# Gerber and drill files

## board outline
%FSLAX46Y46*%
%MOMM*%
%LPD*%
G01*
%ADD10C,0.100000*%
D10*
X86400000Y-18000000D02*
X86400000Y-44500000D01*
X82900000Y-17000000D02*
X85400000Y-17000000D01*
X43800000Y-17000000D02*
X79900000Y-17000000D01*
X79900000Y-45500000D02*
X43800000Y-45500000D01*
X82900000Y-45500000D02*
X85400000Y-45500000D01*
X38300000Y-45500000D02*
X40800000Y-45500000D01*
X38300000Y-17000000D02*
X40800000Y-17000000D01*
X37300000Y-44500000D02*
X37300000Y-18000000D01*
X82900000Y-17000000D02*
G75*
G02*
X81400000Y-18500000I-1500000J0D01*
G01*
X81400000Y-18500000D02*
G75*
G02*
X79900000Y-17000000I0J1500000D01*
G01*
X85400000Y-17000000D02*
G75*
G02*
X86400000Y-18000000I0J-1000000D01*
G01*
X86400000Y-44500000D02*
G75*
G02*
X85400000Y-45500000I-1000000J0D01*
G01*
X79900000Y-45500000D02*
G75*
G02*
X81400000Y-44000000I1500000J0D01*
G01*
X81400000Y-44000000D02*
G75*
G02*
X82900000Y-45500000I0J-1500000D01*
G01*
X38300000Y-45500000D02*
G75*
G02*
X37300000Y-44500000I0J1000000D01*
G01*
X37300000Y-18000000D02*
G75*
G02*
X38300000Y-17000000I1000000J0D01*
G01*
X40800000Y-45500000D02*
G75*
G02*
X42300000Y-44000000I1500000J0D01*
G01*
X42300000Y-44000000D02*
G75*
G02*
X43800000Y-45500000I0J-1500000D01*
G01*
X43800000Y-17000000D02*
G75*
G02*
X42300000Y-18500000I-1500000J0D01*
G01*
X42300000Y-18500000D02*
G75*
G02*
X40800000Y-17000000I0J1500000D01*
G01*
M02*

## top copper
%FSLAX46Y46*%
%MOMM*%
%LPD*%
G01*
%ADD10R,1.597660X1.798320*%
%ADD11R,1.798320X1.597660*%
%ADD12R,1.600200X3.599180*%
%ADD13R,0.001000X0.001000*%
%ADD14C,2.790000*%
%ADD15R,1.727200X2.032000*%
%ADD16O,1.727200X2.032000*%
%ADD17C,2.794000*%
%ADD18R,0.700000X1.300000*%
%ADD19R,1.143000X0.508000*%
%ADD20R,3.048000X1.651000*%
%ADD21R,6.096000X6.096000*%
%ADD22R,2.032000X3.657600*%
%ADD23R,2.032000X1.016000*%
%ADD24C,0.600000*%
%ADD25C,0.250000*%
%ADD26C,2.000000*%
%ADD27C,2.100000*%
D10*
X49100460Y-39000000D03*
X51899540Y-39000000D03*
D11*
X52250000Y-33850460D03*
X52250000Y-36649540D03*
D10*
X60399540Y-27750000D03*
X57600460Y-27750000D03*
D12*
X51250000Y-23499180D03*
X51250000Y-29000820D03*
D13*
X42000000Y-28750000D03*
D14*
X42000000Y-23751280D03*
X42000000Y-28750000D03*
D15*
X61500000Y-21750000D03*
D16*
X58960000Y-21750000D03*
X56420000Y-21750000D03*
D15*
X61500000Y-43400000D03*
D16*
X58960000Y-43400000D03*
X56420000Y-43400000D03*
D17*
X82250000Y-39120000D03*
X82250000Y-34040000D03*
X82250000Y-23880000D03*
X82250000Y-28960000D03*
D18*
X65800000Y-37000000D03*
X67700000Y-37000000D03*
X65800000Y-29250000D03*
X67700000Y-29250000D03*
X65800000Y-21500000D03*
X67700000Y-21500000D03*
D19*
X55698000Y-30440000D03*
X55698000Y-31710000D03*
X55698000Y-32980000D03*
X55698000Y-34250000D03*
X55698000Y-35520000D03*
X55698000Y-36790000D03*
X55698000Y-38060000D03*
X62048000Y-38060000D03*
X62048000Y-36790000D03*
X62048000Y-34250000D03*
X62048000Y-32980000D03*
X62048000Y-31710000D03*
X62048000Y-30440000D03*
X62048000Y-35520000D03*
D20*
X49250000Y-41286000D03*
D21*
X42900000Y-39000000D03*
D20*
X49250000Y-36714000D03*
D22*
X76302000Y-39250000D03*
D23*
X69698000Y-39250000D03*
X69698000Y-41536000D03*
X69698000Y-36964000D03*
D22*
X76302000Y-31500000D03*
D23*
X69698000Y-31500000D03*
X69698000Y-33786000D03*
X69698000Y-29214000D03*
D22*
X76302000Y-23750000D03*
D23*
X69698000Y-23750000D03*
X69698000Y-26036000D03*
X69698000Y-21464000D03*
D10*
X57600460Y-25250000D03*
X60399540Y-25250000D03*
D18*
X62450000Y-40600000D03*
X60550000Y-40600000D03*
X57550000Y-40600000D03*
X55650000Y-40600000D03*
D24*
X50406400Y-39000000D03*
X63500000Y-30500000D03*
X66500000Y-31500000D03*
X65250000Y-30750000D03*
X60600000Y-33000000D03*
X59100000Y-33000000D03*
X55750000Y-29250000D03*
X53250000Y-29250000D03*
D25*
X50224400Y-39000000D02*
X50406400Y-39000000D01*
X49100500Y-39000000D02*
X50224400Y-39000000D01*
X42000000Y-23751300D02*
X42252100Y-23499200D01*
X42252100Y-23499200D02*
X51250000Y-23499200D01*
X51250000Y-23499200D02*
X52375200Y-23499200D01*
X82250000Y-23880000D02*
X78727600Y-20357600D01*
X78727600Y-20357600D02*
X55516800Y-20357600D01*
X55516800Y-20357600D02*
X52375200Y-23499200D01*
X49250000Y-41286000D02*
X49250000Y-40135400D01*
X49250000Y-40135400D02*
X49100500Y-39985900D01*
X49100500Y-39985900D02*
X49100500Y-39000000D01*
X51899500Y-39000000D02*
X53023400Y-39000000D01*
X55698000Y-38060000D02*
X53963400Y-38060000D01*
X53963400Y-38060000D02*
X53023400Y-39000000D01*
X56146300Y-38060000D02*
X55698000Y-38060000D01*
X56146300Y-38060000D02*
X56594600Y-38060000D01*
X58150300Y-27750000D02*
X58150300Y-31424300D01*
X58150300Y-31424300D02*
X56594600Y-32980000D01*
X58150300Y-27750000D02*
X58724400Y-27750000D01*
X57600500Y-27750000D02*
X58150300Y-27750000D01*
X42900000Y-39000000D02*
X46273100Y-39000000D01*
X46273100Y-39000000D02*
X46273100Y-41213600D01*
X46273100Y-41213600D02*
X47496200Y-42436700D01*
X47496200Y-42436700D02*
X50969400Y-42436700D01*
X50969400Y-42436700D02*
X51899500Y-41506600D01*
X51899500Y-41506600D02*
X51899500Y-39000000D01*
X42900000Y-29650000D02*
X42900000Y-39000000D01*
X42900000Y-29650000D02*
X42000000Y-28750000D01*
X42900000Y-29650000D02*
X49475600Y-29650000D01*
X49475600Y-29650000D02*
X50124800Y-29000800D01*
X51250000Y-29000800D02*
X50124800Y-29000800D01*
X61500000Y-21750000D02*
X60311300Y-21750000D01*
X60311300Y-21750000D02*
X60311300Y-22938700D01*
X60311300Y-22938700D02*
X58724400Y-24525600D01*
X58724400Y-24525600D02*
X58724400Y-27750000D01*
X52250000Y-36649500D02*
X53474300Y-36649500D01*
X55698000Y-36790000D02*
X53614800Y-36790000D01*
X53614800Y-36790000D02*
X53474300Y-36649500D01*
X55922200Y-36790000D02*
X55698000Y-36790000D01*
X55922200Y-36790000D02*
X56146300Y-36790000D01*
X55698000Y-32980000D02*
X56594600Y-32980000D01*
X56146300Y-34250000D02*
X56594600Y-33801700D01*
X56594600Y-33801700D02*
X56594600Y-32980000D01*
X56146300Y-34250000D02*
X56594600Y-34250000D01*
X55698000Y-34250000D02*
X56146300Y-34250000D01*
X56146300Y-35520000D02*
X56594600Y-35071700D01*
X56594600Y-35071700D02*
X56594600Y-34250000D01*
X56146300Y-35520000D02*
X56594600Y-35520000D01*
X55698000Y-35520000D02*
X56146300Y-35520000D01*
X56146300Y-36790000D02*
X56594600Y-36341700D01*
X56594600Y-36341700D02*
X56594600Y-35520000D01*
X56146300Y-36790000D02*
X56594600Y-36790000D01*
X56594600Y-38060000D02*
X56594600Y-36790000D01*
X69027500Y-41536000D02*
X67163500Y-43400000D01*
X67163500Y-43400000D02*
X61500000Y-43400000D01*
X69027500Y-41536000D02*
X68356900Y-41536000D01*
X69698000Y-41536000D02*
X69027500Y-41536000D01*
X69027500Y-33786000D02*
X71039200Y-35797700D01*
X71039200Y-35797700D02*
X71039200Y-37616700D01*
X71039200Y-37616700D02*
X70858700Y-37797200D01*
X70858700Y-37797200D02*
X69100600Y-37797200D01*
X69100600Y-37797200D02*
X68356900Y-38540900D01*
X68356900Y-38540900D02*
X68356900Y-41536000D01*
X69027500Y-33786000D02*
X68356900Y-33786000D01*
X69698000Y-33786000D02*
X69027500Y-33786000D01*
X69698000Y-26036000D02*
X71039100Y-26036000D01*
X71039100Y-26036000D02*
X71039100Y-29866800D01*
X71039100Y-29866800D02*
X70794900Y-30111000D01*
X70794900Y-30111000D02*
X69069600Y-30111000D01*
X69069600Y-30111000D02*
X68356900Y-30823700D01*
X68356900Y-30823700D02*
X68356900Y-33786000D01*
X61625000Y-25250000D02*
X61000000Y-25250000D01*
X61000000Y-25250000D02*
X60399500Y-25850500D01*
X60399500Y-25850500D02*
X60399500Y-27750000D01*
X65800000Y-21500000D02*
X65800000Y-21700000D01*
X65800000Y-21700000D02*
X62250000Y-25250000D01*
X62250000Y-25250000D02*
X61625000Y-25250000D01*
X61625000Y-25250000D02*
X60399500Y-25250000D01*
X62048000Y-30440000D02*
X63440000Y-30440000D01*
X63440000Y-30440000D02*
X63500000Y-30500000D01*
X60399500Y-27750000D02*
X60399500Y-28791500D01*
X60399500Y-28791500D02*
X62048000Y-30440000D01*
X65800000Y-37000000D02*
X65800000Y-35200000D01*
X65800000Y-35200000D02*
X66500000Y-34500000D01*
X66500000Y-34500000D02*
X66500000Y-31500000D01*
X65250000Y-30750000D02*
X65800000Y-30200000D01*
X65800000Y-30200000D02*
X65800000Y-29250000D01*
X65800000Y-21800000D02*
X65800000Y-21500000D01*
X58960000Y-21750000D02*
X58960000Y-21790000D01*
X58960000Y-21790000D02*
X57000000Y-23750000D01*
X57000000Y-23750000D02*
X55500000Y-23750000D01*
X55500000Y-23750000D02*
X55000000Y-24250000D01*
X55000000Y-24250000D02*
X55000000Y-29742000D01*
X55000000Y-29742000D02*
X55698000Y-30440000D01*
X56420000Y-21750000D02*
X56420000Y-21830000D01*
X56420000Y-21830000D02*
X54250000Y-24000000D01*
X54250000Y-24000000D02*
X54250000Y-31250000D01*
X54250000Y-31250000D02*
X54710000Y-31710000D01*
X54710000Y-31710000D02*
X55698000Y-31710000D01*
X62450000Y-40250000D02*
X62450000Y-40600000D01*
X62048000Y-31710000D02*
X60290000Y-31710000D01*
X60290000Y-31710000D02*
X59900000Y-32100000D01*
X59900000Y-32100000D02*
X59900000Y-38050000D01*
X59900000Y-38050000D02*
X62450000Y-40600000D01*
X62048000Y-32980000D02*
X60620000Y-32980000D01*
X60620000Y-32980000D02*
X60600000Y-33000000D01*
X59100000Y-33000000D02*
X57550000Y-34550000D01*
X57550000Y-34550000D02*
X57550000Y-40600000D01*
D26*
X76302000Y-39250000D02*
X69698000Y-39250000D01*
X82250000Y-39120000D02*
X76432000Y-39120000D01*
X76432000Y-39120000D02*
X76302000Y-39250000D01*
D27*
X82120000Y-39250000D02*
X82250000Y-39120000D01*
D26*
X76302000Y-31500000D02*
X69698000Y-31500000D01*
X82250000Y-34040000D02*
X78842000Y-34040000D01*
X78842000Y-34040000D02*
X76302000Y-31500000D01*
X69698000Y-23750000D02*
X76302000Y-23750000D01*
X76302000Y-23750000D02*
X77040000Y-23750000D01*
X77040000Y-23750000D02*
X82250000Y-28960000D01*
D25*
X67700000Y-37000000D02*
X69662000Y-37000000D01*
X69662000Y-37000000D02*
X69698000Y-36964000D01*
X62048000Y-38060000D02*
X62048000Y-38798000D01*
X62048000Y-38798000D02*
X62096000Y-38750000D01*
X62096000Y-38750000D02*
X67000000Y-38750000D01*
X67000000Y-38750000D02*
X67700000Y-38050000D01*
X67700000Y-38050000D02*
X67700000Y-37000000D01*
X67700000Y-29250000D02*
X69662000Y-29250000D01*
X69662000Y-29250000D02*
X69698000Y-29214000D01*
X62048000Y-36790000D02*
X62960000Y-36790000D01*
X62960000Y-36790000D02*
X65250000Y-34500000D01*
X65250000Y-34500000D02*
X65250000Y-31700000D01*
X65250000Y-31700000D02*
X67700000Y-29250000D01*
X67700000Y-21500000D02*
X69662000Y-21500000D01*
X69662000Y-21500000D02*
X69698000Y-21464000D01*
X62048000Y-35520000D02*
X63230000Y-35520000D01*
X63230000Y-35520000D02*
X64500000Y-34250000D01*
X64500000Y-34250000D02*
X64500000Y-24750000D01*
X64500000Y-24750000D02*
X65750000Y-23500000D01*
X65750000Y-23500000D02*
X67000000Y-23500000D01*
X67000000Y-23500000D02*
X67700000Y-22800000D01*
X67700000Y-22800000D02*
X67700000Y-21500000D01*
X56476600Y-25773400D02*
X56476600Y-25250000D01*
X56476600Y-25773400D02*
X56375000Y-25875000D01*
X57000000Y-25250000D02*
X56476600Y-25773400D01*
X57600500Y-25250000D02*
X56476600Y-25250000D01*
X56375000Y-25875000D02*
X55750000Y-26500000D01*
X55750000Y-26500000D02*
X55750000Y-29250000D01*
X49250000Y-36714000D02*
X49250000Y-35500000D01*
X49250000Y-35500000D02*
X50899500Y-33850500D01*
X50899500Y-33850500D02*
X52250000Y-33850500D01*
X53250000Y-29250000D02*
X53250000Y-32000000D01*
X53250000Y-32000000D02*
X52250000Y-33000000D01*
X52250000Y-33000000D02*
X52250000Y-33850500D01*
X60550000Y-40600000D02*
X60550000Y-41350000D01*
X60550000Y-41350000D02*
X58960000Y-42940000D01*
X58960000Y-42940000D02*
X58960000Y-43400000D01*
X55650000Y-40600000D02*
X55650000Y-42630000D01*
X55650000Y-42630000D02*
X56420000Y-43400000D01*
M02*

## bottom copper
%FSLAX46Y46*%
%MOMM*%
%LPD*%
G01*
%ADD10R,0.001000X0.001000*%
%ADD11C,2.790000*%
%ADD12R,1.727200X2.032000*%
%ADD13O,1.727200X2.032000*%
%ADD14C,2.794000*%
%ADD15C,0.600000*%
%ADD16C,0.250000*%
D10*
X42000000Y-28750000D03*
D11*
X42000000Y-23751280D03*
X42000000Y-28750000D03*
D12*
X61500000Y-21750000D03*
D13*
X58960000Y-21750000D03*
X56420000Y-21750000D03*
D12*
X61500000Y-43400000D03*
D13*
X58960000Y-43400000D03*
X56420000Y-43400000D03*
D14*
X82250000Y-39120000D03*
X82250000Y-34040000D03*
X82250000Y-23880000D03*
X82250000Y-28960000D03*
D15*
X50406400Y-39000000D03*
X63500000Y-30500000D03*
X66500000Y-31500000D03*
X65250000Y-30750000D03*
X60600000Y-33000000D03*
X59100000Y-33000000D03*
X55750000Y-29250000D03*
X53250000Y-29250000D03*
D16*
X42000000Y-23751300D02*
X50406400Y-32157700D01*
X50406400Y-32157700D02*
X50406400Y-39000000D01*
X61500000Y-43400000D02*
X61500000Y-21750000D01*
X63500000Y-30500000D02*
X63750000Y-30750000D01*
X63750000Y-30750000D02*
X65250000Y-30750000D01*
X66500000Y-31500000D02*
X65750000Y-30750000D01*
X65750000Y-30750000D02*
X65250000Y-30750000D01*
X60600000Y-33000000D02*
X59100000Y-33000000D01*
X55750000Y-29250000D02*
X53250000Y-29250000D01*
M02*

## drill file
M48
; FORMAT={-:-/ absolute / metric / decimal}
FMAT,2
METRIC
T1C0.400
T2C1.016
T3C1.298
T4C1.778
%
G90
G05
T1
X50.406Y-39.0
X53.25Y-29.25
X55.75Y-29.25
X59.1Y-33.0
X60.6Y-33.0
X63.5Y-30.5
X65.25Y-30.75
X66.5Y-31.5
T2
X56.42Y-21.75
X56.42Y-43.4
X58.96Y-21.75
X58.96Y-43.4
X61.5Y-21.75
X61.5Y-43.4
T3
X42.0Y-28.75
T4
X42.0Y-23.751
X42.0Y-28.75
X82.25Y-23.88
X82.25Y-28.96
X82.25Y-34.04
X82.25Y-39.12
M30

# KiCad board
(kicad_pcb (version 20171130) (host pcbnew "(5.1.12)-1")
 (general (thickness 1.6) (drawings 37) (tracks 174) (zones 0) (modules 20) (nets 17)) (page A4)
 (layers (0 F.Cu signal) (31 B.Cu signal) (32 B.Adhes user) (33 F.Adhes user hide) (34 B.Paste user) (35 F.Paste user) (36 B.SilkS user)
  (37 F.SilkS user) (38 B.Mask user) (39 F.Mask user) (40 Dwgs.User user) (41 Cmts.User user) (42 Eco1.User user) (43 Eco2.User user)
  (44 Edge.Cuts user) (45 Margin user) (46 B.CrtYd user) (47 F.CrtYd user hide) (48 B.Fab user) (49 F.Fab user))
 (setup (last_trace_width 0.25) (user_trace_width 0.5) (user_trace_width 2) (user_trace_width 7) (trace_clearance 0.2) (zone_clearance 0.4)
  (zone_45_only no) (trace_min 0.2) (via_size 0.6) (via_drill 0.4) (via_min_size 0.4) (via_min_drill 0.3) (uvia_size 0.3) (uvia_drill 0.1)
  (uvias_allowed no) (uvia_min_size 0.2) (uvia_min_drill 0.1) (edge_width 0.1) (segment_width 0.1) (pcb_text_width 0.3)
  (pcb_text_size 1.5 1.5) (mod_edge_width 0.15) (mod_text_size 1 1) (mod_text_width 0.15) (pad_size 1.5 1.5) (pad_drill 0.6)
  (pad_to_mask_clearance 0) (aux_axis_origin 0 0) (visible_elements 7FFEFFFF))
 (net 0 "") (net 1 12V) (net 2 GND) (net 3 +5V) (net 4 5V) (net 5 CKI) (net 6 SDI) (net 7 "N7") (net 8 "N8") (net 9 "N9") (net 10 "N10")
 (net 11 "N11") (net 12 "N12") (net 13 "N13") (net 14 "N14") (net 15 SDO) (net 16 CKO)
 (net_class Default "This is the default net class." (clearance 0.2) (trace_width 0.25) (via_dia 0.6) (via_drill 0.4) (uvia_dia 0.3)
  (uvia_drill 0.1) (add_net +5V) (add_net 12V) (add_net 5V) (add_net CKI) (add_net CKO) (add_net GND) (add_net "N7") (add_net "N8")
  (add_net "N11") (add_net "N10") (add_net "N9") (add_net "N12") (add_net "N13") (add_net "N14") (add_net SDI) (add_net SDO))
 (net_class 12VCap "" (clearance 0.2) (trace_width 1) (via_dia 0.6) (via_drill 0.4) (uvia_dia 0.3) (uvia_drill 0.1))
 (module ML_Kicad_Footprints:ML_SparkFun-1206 (layer F.Cu) (at 50.5 39)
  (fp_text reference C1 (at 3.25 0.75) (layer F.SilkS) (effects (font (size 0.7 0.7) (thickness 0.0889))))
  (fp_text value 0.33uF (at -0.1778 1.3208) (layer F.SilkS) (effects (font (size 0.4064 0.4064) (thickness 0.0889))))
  (pad 1 smd rect (at -1.39954 0) (size 1.59766 1.79832) (layers F.Cu F.Paste F.Mask) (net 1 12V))
  (pad 2 smd rect (at 1.39954 0) (size 1.59766 1.79832) (layers F.Cu F.Paste F.Mask) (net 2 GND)))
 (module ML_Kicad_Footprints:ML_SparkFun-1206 (layer F.Cu) (at 52.25 35.25 270)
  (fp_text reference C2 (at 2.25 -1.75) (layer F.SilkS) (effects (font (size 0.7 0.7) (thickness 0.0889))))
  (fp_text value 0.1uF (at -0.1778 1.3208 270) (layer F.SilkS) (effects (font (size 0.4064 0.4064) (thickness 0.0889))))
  (pad 1 smd rect (at -1.39954 0 270) (size 1.59766 1.79832) (layers F.Cu F.Paste F.Mask) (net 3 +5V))
  (pad 2 smd rect (at 1.39954 0 270) (size 1.59766 1.79832) (layers F.Cu F.Paste F.Mask) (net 2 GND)))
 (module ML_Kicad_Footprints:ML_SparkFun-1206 (layer F.Cu) (at 59 27.75 180)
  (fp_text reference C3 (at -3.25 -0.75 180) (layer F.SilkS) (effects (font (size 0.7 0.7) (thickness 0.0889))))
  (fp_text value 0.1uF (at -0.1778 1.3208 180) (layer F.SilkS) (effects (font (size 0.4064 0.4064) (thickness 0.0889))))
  (pad 1 smd rect (at -1.39954 0 180) (size 1.59766 1.79832) (layers F.Cu F.Paste F.Mask) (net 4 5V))
  (pad 2 smd rect (at 1.39954 0 180) (size 1.59766 1.79832) (layers F.Cu F.Paste F.Mask) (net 2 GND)))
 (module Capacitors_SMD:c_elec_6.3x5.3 (layer F.Cu) (at 51.25 26.25 90)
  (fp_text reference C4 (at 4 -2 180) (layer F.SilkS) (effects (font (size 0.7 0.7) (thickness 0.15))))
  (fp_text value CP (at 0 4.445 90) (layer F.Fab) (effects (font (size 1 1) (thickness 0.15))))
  (pad 1 smd rect (at 2.75082 0 90) (size 3.59918 1.6002) (layers F.Cu F.Paste F.Mask) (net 1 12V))
  (pad 2 smd rect (at -2.75082 0 90) (size 3.59918 1.6002) (layers F.Cu F.Paste F.Mask) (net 2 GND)))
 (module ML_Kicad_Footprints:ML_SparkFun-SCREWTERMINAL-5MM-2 (layer F.Cu) (at 42 28.75 90)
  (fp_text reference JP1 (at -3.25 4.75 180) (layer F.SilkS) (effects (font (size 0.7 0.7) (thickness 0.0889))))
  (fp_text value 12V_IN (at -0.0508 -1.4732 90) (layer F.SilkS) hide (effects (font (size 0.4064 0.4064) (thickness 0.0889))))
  (pad 1 thru_hole rect (at 0 0 90) (size 2.032 0) (drill 1.29794) (layers *.Cu F.Paste F.SilkS F.Mask) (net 2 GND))
  (pad 2 thru_hole circle (at 4.99872 0 90) (size 2.79 2.79) (drill 1.778) (layers *.Cu *.Mask F.Paste F.SilkS) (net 1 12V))
  (pad 1 thru_hole circle (at 0 0 90) (size 2.79 2.79) (drill 1.778) (layers *.Cu *.Mask F.Paste F.SilkS) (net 2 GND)))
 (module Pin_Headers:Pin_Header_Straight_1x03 (layer F.Cu) (at 61.5 21.75 270)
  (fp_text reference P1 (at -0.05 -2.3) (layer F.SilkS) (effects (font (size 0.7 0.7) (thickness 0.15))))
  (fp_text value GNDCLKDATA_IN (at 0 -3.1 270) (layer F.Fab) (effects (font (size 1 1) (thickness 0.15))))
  (pad 1 thru_hole rect (at 0 0 270) (size 2.032 1.7272) (drill 1.016) (layers *.Cu *.Mask F.SilkS) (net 2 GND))
  (pad 2 thru_hole oval (at 0 2.54 270) (size 2.032 1.7272) (drill 1.016) (layers *.Cu *.Mask F.SilkS) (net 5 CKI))
  (pad 3 thru_hole oval (at 0 5.08 270) (size 2.032 1.7272) (drill 1.016) (layers *.Cu *.Mask F.SilkS) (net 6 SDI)))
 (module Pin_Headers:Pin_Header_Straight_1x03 (layer F.Cu) (at 61.5 43.4 270)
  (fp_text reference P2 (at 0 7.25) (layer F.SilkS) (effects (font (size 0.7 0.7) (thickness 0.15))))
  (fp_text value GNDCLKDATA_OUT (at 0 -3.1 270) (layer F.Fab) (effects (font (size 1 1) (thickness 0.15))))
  (pad 1 thru_hole rect (at 0 0 270) (size 2.032 1.7272) (drill 1.016) (layers *.Cu *.Mask F.SilkS) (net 2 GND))
  (pad 2 thru_hole oval (at 0 2.54 270) (size 2.032 1.7272) (drill 1.016) (layers *.Cu *.Mask F.SilkS) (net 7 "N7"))
  (pad 3 thru_hole oval (at 0 5.08 270) (size 2.032 1.7272) (drill 1.016) (layers *.Cu *.Mask F.SilkS) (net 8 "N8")))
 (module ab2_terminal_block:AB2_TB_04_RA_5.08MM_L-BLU (layer F.Cu) (at 82.25 31.5 270)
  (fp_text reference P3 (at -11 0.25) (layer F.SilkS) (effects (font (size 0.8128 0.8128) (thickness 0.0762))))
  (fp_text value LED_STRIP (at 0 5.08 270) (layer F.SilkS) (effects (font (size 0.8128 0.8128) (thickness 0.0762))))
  (pad 4 thru_hole circle (at 7.62 0 270) (size 2.794 2.794) (drill 1.778) (layers *.Cu *.Mask F.SilkS) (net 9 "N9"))
  (pad 3 thru_hole circle (at 2.54 0 270) (size 2.794 2.794) (drill 1.778) (layers *.Cu *.Mask F.SilkS) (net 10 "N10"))
  (pad 1 thru_hole circle (at -7.62 0 270) (size 2.794 2.794) (drill 1.778) (layers *.Cu *.Mask F.SilkS) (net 1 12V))
  (pad 2 thru_hole circle (at -2.54 0 270) (size 2.794 2.794) (drill 1.778) (layers *.Cu *.Mask F.SilkS) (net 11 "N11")))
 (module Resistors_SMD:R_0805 (layer F.Cu) (at 66.75 37)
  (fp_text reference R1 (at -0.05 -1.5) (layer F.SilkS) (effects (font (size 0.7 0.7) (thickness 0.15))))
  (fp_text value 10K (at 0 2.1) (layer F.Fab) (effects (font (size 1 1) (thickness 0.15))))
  (pad 1 smd rect (at -0.95 0) (size 0.7 1.3) (layers F.Cu F.Paste F.Mask) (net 4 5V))
  (pad 2 smd rect (at 0.95 0) (size 0.7 1.3) (layers F.Cu F.Paste F.Mask) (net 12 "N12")))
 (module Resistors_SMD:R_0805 (layer F.Cu) (at 66.75 29.25)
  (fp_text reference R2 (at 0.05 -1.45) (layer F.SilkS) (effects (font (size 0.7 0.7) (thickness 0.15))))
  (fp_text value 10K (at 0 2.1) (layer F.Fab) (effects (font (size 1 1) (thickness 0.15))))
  (pad 1 smd rect (at -0.95 0) (size 0.7 1.3) (layers F.Cu F.Paste F.Mask) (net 4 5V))
  (pad 2 smd rect (at 0.95 0) (size 0.7 1.3) (layers F.Cu F.Paste F.Mask) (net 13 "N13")))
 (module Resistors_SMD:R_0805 (layer F.Cu) (at 66.75 21.5)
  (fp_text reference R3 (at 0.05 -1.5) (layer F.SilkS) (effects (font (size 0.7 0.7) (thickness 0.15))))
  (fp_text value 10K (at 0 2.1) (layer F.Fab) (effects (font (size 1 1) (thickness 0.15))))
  (pad 1 smd rect (at -0.95 0) (size 0.7 1.3) (layers F.Cu F.Paste F.Mask) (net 4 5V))
  (pad 2 smd rect (at 0.95 0) (size 0.7 1.3) (layers F.Cu F.Paste F.Mask) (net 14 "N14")))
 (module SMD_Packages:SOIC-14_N (layer F.Cu) (at 59 34.25 270)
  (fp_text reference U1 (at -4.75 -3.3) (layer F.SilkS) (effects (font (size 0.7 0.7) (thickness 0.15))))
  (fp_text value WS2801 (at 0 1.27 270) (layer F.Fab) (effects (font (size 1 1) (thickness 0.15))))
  (pad 1 smd rect (at -3.81 3.302 270) (size 0.508 1.143) (layers F.Cu F.Paste F.Mask) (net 5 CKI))
  (pad 2 smd rect (at -2.54 3.302 270) (size 0.508 1.143) (layers F.Cu F.Paste F.Mask) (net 6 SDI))
  (pad 3 smd rect (at -1.27 3.302 270) (size 0.508 1.143) (layers F.Cu F.Paste F.Mask) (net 2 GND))
  (pad 4 smd rect (at 0 3.302 270) (size 0.508 1.143) (layers F.Cu F.Paste F.Mask) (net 2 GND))
  (pad 5 smd rect (at 1.27 3.302 270) (size 0.508 1.143) (layers F.Cu F.Paste F.Mask) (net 2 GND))
  (pad 6 smd rect (at 2.54 3.302 270) (size 0.508 1.143) (layers F.Cu F.Paste F.Mask) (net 2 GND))
  (pad 7 smd rect (at 3.81 3.302 270) (size 0.508 1.143) (layers F.Cu F.Paste F.Mask) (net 2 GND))
  (pad 8 smd rect (at 3.81 -3.048 270) (size 0.508 1.143) (layers F.Cu F.Paste F.Mask) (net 12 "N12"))
  (pad 9 smd rect (at 2.54 -3.048 270) (size 0.508 1.143) (layers F.Cu F.Paste F.Mask) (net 13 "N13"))
  (pad 11 smd rect (at 0 -3.048 270) (size 0.508 1.143) (layers F.Cu F.Paste F.Mask))
  (pad 12 smd rect (at -1.27 -3.048 270) (size 0.508 1.143) (layers F.Cu F.Paste F.Mask) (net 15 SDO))
  (pad 13 smd rect (at -2.54 -3.048 270) (size 0.508 1.143) (layers F.Cu F.Paste F.Mask) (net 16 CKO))
  (pad 14 smd rect (at -3.81 -3.048 270) (size 0.508 1.143) (layers F.Cu F.Paste F.Mask) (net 4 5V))
  (pad 10 smd rect (at 1.27 -3.048 270) (size 0.508 1.143) (layers F.Cu F.Paste F.Mask) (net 14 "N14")))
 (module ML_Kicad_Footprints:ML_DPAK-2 (layer F.Cu) (at 49.25 39 90)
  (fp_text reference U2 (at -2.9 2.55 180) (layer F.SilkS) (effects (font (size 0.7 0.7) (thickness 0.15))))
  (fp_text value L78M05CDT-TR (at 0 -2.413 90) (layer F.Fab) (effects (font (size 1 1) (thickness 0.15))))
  (pad VI smd rect (at -2.286 0 90) (size 1.651 3.048) (layers F.Cu F.Paste F.Mask) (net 1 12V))
  (pad GND smd rect (at 0 -6.35 90) (size 6.096 6.096) (layers F.Cu F.Paste F.Mask) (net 2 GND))
  (pad VO smd rect (at 2.286 0 90) (size 1.651 3.048) (layers F.Cu F.Paste F.Mask) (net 3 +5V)))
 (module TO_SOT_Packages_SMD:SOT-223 (layer F.Cu) (at 73 39.25 270)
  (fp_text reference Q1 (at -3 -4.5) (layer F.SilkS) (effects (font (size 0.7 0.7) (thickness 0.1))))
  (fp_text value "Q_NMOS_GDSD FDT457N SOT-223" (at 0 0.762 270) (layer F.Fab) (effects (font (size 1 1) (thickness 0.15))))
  (pad 4 smd rect (at 0 -3.302 270) (size 3.6576 2.032) (layers F.Cu F.Paste F.Mask) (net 9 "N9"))
  (pad 2 smd rect (at 0 3.302 270) (size 1.016 2.032) (layers F.Cu F.Paste F.Mask) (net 9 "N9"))
  (pad 3 smd rect (at 2.286 3.302 270) (size 1.016 2.032) (layers F.Cu F.Paste F.Mask) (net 2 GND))
  (pad 1 smd rect (at -2.286 3.302 270) (size 1.016 2.032) (layers F.Cu F.Paste F.Mask) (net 12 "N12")))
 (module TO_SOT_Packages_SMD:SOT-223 (layer F.Cu) (at 73 31.5 270)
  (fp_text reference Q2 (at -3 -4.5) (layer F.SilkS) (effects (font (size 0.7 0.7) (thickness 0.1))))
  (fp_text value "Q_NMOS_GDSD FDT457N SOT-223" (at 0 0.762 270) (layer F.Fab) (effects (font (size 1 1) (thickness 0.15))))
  (pad 4 smd rect (at 0 -3.302 270) (size 3.6576 2.032) (layers F.Cu F.Paste F.Mask) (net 10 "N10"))
  (pad 2 smd rect (at 0 3.302 270) (size 1.016 2.032) (layers F.Cu F.Paste F.Mask) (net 10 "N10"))
  (pad 3 smd rect (at 2.286 3.302 270) (size 1.016 2.032) (layers F.Cu F.Paste F.Mask) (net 2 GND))
  (pad 1 smd rect (at -2.286 3.302 270) (size 1.016 2.032) (layers F.Cu F.Paste F.Mask) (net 13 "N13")))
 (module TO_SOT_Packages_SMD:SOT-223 (layer F.Cu) (at 73 23.75 270)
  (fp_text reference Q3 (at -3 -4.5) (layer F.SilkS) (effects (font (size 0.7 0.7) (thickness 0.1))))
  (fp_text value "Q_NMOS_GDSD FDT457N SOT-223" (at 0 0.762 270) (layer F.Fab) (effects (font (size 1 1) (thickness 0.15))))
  (pad 4 smd rect (at 0 -3.302 270) (size 3.6576 2.032) (layers F.Cu F.Paste F.Mask) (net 11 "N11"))
  (pad 2 smd rect (at 0 3.302 270) (size 1.016 2.032) (layers F.Cu F.Paste F.Mask) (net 11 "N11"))
  (pad 3 smd rect (at 2.286 3.302 270) (size 1.016 2.032) (layers F.Cu F.Paste F.Mask) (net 2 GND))
  (pad 1 smd rect (at -2.286 3.302 270) (size 1.016 2.032) (layers F.Cu F.Paste F.Mask) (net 14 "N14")))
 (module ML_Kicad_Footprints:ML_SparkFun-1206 (layer F.Cu) (at 59 25.25)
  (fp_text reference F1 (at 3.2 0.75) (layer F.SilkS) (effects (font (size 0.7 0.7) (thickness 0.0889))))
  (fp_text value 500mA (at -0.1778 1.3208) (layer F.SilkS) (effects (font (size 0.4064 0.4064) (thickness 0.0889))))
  (pad 1 smd rect (at -1.39954 0) (size 1.59766 1.79832) (layers F.Cu F.Paste F.Mask) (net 3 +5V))
  (pad 2 smd rect (at 1.39954 0) (size 1.59766 1.79832) (layers F.Cu F.Paste F.Mask) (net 4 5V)))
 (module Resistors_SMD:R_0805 (layer F.Cu) (at 61.5 40.6 180)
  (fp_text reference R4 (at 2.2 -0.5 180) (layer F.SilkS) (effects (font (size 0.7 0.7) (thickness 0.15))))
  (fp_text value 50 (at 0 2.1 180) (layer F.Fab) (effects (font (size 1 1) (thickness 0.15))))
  (pad 1 smd rect (at -0.95 0 180) (size 0.7 1.3) (layers F.Cu F.Paste F.Mask) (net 16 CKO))
  (pad 2 smd rect (at 0.95 0 180) (size 0.7 1.3) (layers F.Cu F.Paste F.Mask) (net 7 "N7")))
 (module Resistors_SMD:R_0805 (layer F.Cu) (at 56.6 40.6 180)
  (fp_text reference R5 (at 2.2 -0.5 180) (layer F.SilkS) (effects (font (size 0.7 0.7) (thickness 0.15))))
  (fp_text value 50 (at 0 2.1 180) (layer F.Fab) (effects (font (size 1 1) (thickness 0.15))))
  (pad 1 smd rect (at -0.95 0 180) (size 0.7 1.3) (layers F.Cu F.Paste F.Mask) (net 15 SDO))
  (pad 2 smd rect (at 0.95 0 180) (size 0.7 1.3) (layers F.Cu F.Paste F.Mask) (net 8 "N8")))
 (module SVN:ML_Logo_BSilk (layer F.Cu) (at 42.7 37.25)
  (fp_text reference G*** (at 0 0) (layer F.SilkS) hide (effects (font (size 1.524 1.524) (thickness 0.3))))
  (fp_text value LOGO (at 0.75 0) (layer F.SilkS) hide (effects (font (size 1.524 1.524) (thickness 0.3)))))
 (gr_line (start 86.4 18) (end 86.4 44.5) (angle 90) (layer Edge.Cuts) (width 0.1))
 (gr_line (start 82.9 17) (end 85.4 17) (angle 90) (layer Edge.Cuts) (width 0.1))
 (gr_line (start 43.8 17) (end 79.9 17) (angle 90) (layer Edge.Cuts) (width 0.1))
 (gr_line (start 79.9 45.5) (end 43.8 45.5) (angle 90) (layer Edge.Cuts) (width 0.1))
 (gr_line (start 82.9 45.5) (end 85.4 45.5) (angle 90) (layer Edge.Cuts) (width 0.1))
 (gr_line (start 38.3 45.5) (end 40.8 45.5) (angle 90) (layer Edge.Cuts) (width 0.1))
 (gr_line (start 38.3 17) (end 40.8 17) (angle 90) (layer Edge.Cuts) (width 0.1))
 (gr_line (start 37.3 44.5) (end 37.3 18) (angle 90) (layer Edge.Cuts) (width 0.1))
 (gr_arc (start 81.4 17) (end 82.9 17) (angle 90) (layer Edge.Cuts) (width 0.1))
 (gr_arc (start 81.4 17) (end 81.4 18.5) (angle 90) (layer Edge.Cuts) (width 0.1))
 (gr_arc (start 85.4 18) (end 85.4 17) (angle 90) (layer Edge.Cuts) (width 0.1))
 (gr_arc (start 85.4 44.5) (end 86.4 44.5) (angle 90) (layer Edge.Cuts) (width 0.1))
 (gr_arc (start 81.4 45.5) (end 79.9 45.5) (angle 90) (layer Edge.Cuts) (width 0.1))
 (gr_arc (start 81.4 45.5) (end 81.4 44) (angle 90) (layer Edge.Cuts) (width 0.1))
 (gr_arc (start 38.3 44.5) (end 38.3 45.5) (angle 90) (layer Edge.Cuts) (width 0.1))
 (gr_arc (start 38.3 18) (end 37.3 18) (angle 90) (layer Edge.Cuts) (width 0.1))
 (gr_arc (start 42.3 45.5) (end 40.8 45.5) (angle 90) (layer Edge.Cuts) (width 0.1))
 (gr_arc (start 42.3 45.5) (end 42.3 44) (angle 90) (layer Edge.Cuts) (width 0.1))
 (gr_arc (start 42.3 17) (end 43.8 17) (angle 90) (layer Edge.Cuts) (width 0.1))
 (gr_arc (start 42.3 17) (end 42.3 18.5) (angle 90) (layer Edge.Cuts) (width 0.1))
 (segment (start 50.2244 39) (end 50.4064 39) (width 0.25) (layer F.Cu) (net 1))
 (segment (start 42 23.7513) (end 50.4064 32.1577) (width 0.25) (layer B.Cu) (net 1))
 (segment (start 50.4064 32.1577) (end 50.4064 39) (width 0.25) (layer B.Cu) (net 1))
 (segment (start 49.1005 39) (end 50.2244 39) (width 0.25) (layer F.Cu) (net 1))
 (segment (start 42 23.7513) (end 42.2521 23.4992) (width 0.25) (layer F.Cu) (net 1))
 (segment (start 42.2521 23.4992) (end 51.25 23.4992) (width 0.25) (layer F.Cu) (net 1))
 (segment (start 51.25 23.4992) (end 52.3752 23.4992) (width 0.25) (layer F.Cu) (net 1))
 (segment (start 82.25 23.88) (end 78.7276 20.3576) (width 0.25) (layer F.Cu) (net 1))
 (segment (start 78.7276 20.3576) (end 55.5168 20.3576) (width 0.25) (layer F.Cu) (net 1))
 (segment (start 55.5168 20.3576) (end 52.3752 23.4992) (width 0.25) (layer F.Cu) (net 1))
 (segment (start 49.25 41.286) (end 49.25 40.1354) (width 0.25) (layer F.Cu) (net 1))
 (segment (start 49.25 40.1354) (end 49.1005 39.9859) (width 0.25) (layer F.Cu) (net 1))
 (segment (start 49.1005 39.9859) (end 49.1005 39) (width 0.25) (layer F.Cu) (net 1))
 (via (at 50.4064 39) (size 0.6) (layers F.Cu B.Cu) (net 1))
 (segment (start 51.8995 39) (end 53.0234 39) (width 0.25) (layer F.Cu) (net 2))
 (segment (start 55.698 38.06) (end 53.9634 38.06) (width 0.25) (layer F.Cu) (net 2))
 (segment (start 53.9634 38.06) (end 53.0234 39) (width 0.25) (layer F.Cu) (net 2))
 (segment (start 56.1463 38.06) (end 55.698 38.06) (width 0.25) (layer F.Cu) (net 2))
 (segment (start 56.1463 38.06) (end 56.5946 38.06) (width 0.25) (layer F.Cu) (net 2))
 (segment (start 58.1503 27.75) (end 58.1503 31.4243) (width 0.25) (layer F.Cu) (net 2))
 (segment (start 58.1503 31.4243) (end 56.5946 32.98) (width 0.25) (layer F.Cu) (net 2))
 (segment (start 58.1503 27.75) (end 58.7244 27.75) (width 0.25) (layer F.Cu) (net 2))
 (segment (start 57.6005 27.75) (end 58.1503 27.75) (width 0.25) (layer F.Cu) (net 2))
 (segment (start 42.9 39) (end 46.2731 39) (width 0.25) (layer F.Cu) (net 2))
 (segment (start 46.2731 39) (end 46.2731 41.2136) (width 0.25) (layer F.Cu) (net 2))
 (segment (start 46.2731 41.2136) (end 47.4962 42.4367) (width 0.25) (layer F.Cu) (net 2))
 (segment (start 47.4962 42.4367) (end 50.9694 42.4367) (width 0.25) (layer F.Cu) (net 2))
 (segment (start 50.9694 42.4367) (end 51.8995 41.5066) (width 0.25) (layer F.Cu) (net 2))
 (segment (start 51.8995 41.5066) (end 51.8995 39) (width 0.25) (layer F.Cu) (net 2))
 (segment (start 42.9 29.65) (end 42.9 39) (width 0.25) (layer F.Cu) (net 2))
 (segment (start 42.9 29.65) (end 42 28.75) (width 0.25) (layer F.Cu) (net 2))
 (segment (start 42.9 29.65) (end 49.4756 29.65) (width 0.25) (layer F.Cu) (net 2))
 (segment (start 49.4756 29.65) (end 50.1248 29.0008) (width 0.25) (layer F.Cu) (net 2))
 (segment (start 51.25 29.0008) (end 50.1248 29.0008) (width 0.25) (layer F.Cu) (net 2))
 (segment (start 61.5 21.75) (end 60.3113 21.75) (width 0.25) (layer F.Cu) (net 2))
 (segment (start 60.3113 21.75) (end 60.3113 22.9387) (width 0.25) (layer F.Cu) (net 2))
 (segment (start 60.3113 22.9387) (end 58.7244 24.5256) (width 0.25) (layer F.Cu) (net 2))
 (segment (start 58.7244 24.5256) (end 58.7244 27.75) (width 0.25) (layer F.Cu) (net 2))
 (segment (start 61.5 43.4) (end 61.5 21.75) (width 0.25) (layer B.Cu) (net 2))
 (segment (start 52.25 36.6495) (end 53.4743 36.6495) (width 0.25) (layer F.Cu) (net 2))
 (segment (start 55.698 36.79) (end 53.6148 36.79) (width 0.25) (layer F.Cu) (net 2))
 (segment (start 53.6148 36.79) (end 53.4743 36.6495) (width 0.25) (layer F.Cu) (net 2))
 (segment (start 55.9222 36.79) (end 55.698 36.79) (width 0.25) (layer F.Cu) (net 2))
 (segment (start 55.9222 36.79) (end 56.1463 36.79) (width 0.25) (layer F.Cu) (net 2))
 (segment (start 55.698 32.98) (end 56.5946 32.98) (width 0.25) (layer F.Cu) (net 2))
 (segment (start 56.1463 34.25) (end 56.5946 33.8017) (width 0.25) (layer F.Cu) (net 2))
 (segment (start 56.5946 33.8017) (end 56.5946 32.98) (width 0.25) (layer F.Cu) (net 2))
 (segment (start 56.1463 34.25) (end 56.5946 34.25) (width 0.25) (layer F.Cu) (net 2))
 (segment (start 55.698 34.25) (end 56.1463 34.25) (width 0.25) (layer F.Cu) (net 2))
 (segment (start 56.1463 35.52) (end 56.5946 35.0717) (width 0.25) (layer F.Cu) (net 2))
 (segment (start 56.5946 35.0717) (end 56.5946 34.25) (width 0.25) (layer F.Cu) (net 2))
 (segment (start 56.1463 35.52) (end 56.5946 35.52) (width 0.25) (layer F.Cu) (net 2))
 (segment (start 55.698 35.52) (end 56.1463 35.52) (width 0.25) (layer F.Cu) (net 2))
 (segment (start 56.1463 36.79) (end 56.5946 36.3417) (width 0.25) (layer F.Cu) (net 2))
 (segment (start 56.5946 36.3417) (end 56.5946 35.52) (width 0.25) (layer F.Cu) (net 2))
 (segment (start 56.1463 36.79) (end 56.5946 36.79) (width 0.25) (layer F.Cu) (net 2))
 (segment (start 56.5946 38.06) (end 56.5946 36.79) (width 0.25) (layer F.Cu) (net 2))
 (segment (start 69.0275 41.536) (end 67.1635 43.4) (width 0.25) (layer F.Cu) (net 2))
 (segment (start 67.1635 43.4) (end 61.5 43.4) (width 0.25) (layer F.Cu) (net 2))
 (segment (start 69.0275 41.536) (end 68.3569 41.536) (width 0.25) (layer F.Cu) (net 2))
 (segment (start 69.698 41.536) (end 69.0275 41.536) (width 0.25) (layer F.Cu) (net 2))
 (segment (start 69.0275 33.786) (end 71.0392 35.7977) (width 0.25) (layer F.Cu) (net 2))
 (segment (start 71.0392 35.7977) (end 71.0392 37.6167) (width 0.25) (layer F.Cu) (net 2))
 (segment (start 71.0392 37.6167) (end 70.8587 37.7972) (width 0.25) (layer F.Cu) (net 2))
 (segment (start 70.8587 37.7972) (end 69.1006 37.7972) (width 0.25) (layer F.Cu) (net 2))
 (segment (start 69.1006 37.7972) (end 68.3569 38.5409) (width 0.25) (layer F.Cu) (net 2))
 (segment (start 68.3569 38.5409) (end 68.3569 41.536) (width 0.25) (layer F.Cu) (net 2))
 (segment (start 69.0275 33.786) (end 68.3569 33.786) (width 0.25) (layer F.Cu) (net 2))
 (segment (start 69.698 33.786) (end 69.0275 33.786) (width 0.25) (layer F.Cu) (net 2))
 (segment (start 69.698 26.036) (end 71.0391 26.036) (width 0.25) (layer F.Cu) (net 2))
 (segment (start 71.0391 26.036) (end 71.0391 29.8668) (width 0.25) (layer F.Cu) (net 2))
 (segment (start 71.0391 29.8668) (end 70.7949 30.111) (width 0.25) (layer F.Cu) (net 2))
 (segment (start 70.7949 30.111) (end 69.0696 30.111) (width 0.25) (layer F.Cu) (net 2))
 (segment (start 69.0696 30.111) (end 68.3569 30.8237) (width 0.25) (layer F.Cu) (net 2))
 (segment (start 68.3569 30.8237) (end 68.3569 33.786) (width 0.25) (layer F.Cu) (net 2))
 (segment (start 61.625 25.25) (end 61 25.25) (width 0.25) (layer F.Cu) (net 4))
 (segment (start 61 25.25) (end 60.3995 25.8505) (width 0.25) (layer F.Cu) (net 4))
 (segment (start 60.3995 25.8505) (end 60.3995 27.75) (width 0.25) (layer F.Cu) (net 4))
 (segment (start 65.8 21.5) (end 65.8 21.7) (width 0.25) (layer F.Cu) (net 4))
 (segment (start 65.8 21.7) (end 62.25 25.25) (width 0.25) (layer F.Cu) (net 4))
 (segment (start 62.25 25.25) (end 61.625 25.25) (width 0.25) (layer F.Cu) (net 4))
 (segment (start 61.625 25.25) (end 60.3995 25.25) (width 0.25) (layer F.Cu) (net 4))
 (segment (start 62.048 30.44) (end 63.44 30.44) (width 0.25) (layer F.Cu) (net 4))
 (segment (start 63.44 30.44) (end 63.5 30.5) (width 0.25) (layer F.Cu) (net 4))
 (segment (start 63.5 30.5) (end 63.75 30.75) (width 0.25) (layer B.Cu) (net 4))
 (segment (start 63.75 30.75) (end 65.25 30.75) (width 0.25) (layer B.Cu) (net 4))
 (segment (start 60.3995 27.75) (end 60.3995 28.7915) (width 0.25) (layer F.Cu) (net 4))
 (segment (start 60.3995 28.7915) (end 62.048 30.44) (width 0.25) (layer F.Cu) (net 4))
 (segment (start 65.8 37) (end 65.8 35.2) (width 0.25) (layer F.Cu) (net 4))
 (segment (start 65.8 35.2) (end 66.5 34.5) (width 0.25) (layer F.Cu) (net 4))
 (segment (start 66.5 34.5) (end 66.5 31.5) (width 0.25) (layer F.Cu) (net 4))
 (segment (start 66.5 31.5) (end 65.75 30.75) (width 0.25) (layer B.Cu) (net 4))
 (segment (start 65.75 30.75) (end 65.25 30.75) (width 0.25) (layer B.Cu) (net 4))
 (segment (start 65.25 30.75) (end 65.8 30.2) (width 0.25) (layer F.Cu) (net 4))
 (segment (start 65.8 30.2) (end 65.8 29.25) (width 0.25) (layer F.Cu) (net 4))
 (segment (start 65.8 21.8) (end 65.8 21.5) (width 0.25) (layer F.Cu) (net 4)) (via (at 63.5 30.5) (size 0.6) (layers F.Cu B.Cu) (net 4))
 (via (at 66.5 31.5) (size 0.6) (layers F.Cu B.Cu) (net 4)) (via (at 65.25 30.75) (size 0.6) (layers F.Cu B.Cu) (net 4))
 (segment (start 58.96 21.75) (end 58.96 21.79) (width 0.25) (layer F.Cu) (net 5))
 (segment (start 58.96 21.79) (end 57 23.75) (width 0.25) (layer F.Cu) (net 5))
 (segment (start 57 23.75) (end 55.5 23.75) (width 0.25) (layer F.Cu) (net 5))
 (segment (start 55.5 23.75) (end 55 24.25) (width 0.25) (layer F.Cu) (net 5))
 (segment (start 55 24.25) (end 55 29.742) (width 0.25) (layer F.Cu) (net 5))
 (segment (start 55 29.742) (end 55.698 30.44) (width 0.25) (layer F.Cu) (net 5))
 (segment (start 56.42 21.75) (end 56.42 21.83) (width 0.25) (layer F.Cu) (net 6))
 (segment (start 56.42 21.83) (end 54.25 24) (width 0.25) (layer F.Cu) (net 6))
 (segment (start 54.25 24) (end 54.25 31.25) (width 0.25) (layer F.Cu) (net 6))
 (segment (start 54.25 31.25) (end 54.71 31.71) (width 0.25) (layer F.Cu) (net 6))
 (segment (start 54.71 31.71) (end 55.698 31.71) (width 0.25) (layer F.Cu) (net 6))
 (segment (start 62.45 40.25) (end 62.45 40.6) (width 0.25) (layer F.Cu) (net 16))
 (segment (start 62.048 31.71) (end 60.29 31.71) (width 0.25) (layer F.Cu) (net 16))
 (segment (start 60.29 31.71) (end 59.9 32.1) (width 0.25) (layer F.Cu) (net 16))
 (segment (start 59.9 32.1) (end 59.9 38.05) (width 0.25) (layer F.Cu) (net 16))
 (segment (start 59.9 38.05) (end 62.45 40.6) (width 0.25) (layer F.Cu) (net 16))
 (segment (start 62.048 32.98) (end 60.62 32.98) (width 0.25) (layer F.Cu) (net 15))
 (segment (start 60.62 32.98) (end 60.6 33) (width 0.25) (layer F.Cu) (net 15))
 (segment (start 60.6 33) (end 59.1 33) (width 0.25) (layer B.Cu) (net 15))
 (segment (start 59.1 33) (end 57.55 34.55) (width 0.25) (layer F.Cu) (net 15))
 (segment (start 57.55 34.55) (end 57.55 40.6) (width 0.25) (layer F.Cu) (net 15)) (via (at 60.6 33) (size 0.6) (layers F.Cu B.Cu) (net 15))
 (via (at 59.1 33) (size 0.6) (layers F.Cu B.Cu) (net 15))
 (segment (start 76.302 39.25) (end 69.698 39.25) (width 2) (layer F.Cu) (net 9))
 (segment (start 82.25 39.12) (end 76.432 39.12) (width 2) (layer F.Cu) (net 9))
 (segment (start 76.432 39.12) (end 76.302 39.25) (width 2) (layer F.Cu) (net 9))
 (segment (start 82.12 39.25) (end 82.25 39.12) (width 2.1) (layer F.Cu) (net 9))
 (segment (start 76.302 31.5) (end 69.698 31.5) (width 2) (layer F.Cu) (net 10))
 (segment (start 82.25 34.04) (end 78.842 34.04) (width 2) (layer F.Cu) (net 10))
 (segment (start 78.842 34.04) (end 76.302 31.5) (width 2) (layer F.Cu) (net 10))
 (segment (start 69.698 23.75) (end 76.302 23.75) (width 2) (layer F.Cu) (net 11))
 (segment (start 76.302 23.75) (end 77.04 23.75) (width 2) (layer F.Cu) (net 11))
 (segment (start 77.04 23.75) (end 82.25 28.96) (width 2) (layer F.Cu) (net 11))
 (segment (start 67.7 37) (end 69.662 37) (width 0.25) (layer F.Cu) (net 12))
 (segment (start 69.662 37) (end 69.698 36.964) (width 0.25) (layer F.Cu) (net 12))
 (segment (start 62.048 38.06) (end 62.048 38.798) (width 0.25) (layer F.Cu) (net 12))
 (segment (start 62.048 38.798) (end 62.096 38.75) (width 0.25) (layer F.Cu) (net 12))
 (segment (start 62.096 38.75) (end 67 38.75) (width 0.25) (layer F.Cu) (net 12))
 (segment (start 67 38.75) (end 67.7 38.05) (width 0.25) (layer F.Cu) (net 12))
 (segment (start 67.7 38.05) (end 67.7 37) (width 0.25) (layer F.Cu) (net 12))
 (segment (start 67.7 29.25) (end 69.662 29.25) (width 0.25) (layer F.Cu) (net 13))
 (segment (start 69.662 29.25) (end 69.698 29.214) (width 0.25) (layer F.Cu) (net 13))
 (segment (start 62.048 36.79) (end 62.96 36.79) (width 0.25) (layer F.Cu) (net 13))
 (segment (start 62.96 36.79) (end 65.25 34.5) (width 0.25) (layer F.Cu) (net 13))
 (segment (start 65.25 34.5) (end 65.25 31.7) (width 0.25) (layer F.Cu) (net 13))
 (segment (start 65.25 31.7) (end 67.7 29.25) (width 0.25) (layer F.Cu) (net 13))
 (segment (start 67.7 21.5) (end 69.662 21.5) (width 0.25) (layer F.Cu) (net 14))
 (segment (start 69.662 21.5) (end 69.698 21.464) (width 0.25) (layer F.Cu) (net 14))
 (segment (start 62.048 35.52) (end 63.23 35.52) (width 0.25) (layer F.Cu) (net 14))
 (segment (start 63.23 35.52) (end 64.5 34.25) (width 0.25) (layer F.Cu) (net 14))
 (segment (start 64.5 34.25) (end 64.5 24.75) (width 0.25) (layer F.Cu) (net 14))
 (segment (start 64.5 24.75) (end 65.75 23.5) (width 0.25) (layer F.Cu) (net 14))
 (segment (start 65.75 23.5) (end 67 23.5) (width 0.25) (layer F.Cu) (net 14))
 (segment (start 67 23.5) (end 67.7 22.8) (width 0.25) (layer F.Cu) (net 14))
 (segment (start 67.7 22.8) (end 67.7 21.5) (width 0.25) (layer F.Cu) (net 14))
 (segment (start 56.4766 25.7734) (end 56.4766 25.25) (width 0.25) (layer F.Cu) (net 3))
 (segment (start 56.4766 25.7734) (end 56.375 25.875) (width 0.25) (layer F.Cu) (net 3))
 (segment (start 57 25.25) (end 56.4766 25.7734) (width 0.25) (layer F.Cu) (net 3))
 (segment (start 57.6005 25.25) (end 56.4766 25.25) (width 0.25) (layer F.Cu) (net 3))
 (segment (start 56.375 25.875) (end 55.75 26.5) (width 0.25) (layer F.Cu) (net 3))
 (segment (start 55.75 26.5) (end 55.75 29.25) (width 0.25) (layer F.Cu) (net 3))
 (segment (start 49.25 36.714) (end 49.25 35.5) (width 0.25) (layer F.Cu) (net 3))
 (segment (start 49.25 35.5) (end 50.8995 33.8505) (width 0.25) (layer F.Cu) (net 3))
 (segment (start 50.8995 33.8505) (end 52.25 33.8505) (width 0.25) (layer F.Cu) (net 3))
 (segment (start 55.75 29.25) (end 53.25 29.25) (width 0.25) (layer B.Cu) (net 3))
 (segment (start 53.25 29.25) (end 53.25 32) (width 0.25) (layer F.Cu) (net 3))
 (segment (start 53.25 32) (end 52.25 33) (width 0.25) (layer F.Cu) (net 3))
 (segment (start 52.25 33) (end 52.25 33.8505) (width 0.25) (layer F.Cu) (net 3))
 (via (at 55.75 29.25) (size 0.6) (layers F.Cu B.Cu) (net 3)) (via (at 53.25 29.25) (size 0.6) (layers F.Cu B.Cu) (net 3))
 (segment (start 60.55 40.6) (end 60.55 41.35) (width 0.25) (layer F.Cu) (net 7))
 (segment (start 60.55 41.35) (end 58.96 42.94) (width 0.25) (layer F.Cu) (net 7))
 (segment (start 58.96 42.94) (end 58.96 43.4) (width 0.25) (layer F.Cu) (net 7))
 (segment (start 55.65 40.6) (end 55.65 42.63) (width 0.25) (layer F.Cu) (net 8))
 (segment (start 55.65 42.63) (end 56.42 43.4) (width 0.25) (layer F.Cu) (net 8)))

